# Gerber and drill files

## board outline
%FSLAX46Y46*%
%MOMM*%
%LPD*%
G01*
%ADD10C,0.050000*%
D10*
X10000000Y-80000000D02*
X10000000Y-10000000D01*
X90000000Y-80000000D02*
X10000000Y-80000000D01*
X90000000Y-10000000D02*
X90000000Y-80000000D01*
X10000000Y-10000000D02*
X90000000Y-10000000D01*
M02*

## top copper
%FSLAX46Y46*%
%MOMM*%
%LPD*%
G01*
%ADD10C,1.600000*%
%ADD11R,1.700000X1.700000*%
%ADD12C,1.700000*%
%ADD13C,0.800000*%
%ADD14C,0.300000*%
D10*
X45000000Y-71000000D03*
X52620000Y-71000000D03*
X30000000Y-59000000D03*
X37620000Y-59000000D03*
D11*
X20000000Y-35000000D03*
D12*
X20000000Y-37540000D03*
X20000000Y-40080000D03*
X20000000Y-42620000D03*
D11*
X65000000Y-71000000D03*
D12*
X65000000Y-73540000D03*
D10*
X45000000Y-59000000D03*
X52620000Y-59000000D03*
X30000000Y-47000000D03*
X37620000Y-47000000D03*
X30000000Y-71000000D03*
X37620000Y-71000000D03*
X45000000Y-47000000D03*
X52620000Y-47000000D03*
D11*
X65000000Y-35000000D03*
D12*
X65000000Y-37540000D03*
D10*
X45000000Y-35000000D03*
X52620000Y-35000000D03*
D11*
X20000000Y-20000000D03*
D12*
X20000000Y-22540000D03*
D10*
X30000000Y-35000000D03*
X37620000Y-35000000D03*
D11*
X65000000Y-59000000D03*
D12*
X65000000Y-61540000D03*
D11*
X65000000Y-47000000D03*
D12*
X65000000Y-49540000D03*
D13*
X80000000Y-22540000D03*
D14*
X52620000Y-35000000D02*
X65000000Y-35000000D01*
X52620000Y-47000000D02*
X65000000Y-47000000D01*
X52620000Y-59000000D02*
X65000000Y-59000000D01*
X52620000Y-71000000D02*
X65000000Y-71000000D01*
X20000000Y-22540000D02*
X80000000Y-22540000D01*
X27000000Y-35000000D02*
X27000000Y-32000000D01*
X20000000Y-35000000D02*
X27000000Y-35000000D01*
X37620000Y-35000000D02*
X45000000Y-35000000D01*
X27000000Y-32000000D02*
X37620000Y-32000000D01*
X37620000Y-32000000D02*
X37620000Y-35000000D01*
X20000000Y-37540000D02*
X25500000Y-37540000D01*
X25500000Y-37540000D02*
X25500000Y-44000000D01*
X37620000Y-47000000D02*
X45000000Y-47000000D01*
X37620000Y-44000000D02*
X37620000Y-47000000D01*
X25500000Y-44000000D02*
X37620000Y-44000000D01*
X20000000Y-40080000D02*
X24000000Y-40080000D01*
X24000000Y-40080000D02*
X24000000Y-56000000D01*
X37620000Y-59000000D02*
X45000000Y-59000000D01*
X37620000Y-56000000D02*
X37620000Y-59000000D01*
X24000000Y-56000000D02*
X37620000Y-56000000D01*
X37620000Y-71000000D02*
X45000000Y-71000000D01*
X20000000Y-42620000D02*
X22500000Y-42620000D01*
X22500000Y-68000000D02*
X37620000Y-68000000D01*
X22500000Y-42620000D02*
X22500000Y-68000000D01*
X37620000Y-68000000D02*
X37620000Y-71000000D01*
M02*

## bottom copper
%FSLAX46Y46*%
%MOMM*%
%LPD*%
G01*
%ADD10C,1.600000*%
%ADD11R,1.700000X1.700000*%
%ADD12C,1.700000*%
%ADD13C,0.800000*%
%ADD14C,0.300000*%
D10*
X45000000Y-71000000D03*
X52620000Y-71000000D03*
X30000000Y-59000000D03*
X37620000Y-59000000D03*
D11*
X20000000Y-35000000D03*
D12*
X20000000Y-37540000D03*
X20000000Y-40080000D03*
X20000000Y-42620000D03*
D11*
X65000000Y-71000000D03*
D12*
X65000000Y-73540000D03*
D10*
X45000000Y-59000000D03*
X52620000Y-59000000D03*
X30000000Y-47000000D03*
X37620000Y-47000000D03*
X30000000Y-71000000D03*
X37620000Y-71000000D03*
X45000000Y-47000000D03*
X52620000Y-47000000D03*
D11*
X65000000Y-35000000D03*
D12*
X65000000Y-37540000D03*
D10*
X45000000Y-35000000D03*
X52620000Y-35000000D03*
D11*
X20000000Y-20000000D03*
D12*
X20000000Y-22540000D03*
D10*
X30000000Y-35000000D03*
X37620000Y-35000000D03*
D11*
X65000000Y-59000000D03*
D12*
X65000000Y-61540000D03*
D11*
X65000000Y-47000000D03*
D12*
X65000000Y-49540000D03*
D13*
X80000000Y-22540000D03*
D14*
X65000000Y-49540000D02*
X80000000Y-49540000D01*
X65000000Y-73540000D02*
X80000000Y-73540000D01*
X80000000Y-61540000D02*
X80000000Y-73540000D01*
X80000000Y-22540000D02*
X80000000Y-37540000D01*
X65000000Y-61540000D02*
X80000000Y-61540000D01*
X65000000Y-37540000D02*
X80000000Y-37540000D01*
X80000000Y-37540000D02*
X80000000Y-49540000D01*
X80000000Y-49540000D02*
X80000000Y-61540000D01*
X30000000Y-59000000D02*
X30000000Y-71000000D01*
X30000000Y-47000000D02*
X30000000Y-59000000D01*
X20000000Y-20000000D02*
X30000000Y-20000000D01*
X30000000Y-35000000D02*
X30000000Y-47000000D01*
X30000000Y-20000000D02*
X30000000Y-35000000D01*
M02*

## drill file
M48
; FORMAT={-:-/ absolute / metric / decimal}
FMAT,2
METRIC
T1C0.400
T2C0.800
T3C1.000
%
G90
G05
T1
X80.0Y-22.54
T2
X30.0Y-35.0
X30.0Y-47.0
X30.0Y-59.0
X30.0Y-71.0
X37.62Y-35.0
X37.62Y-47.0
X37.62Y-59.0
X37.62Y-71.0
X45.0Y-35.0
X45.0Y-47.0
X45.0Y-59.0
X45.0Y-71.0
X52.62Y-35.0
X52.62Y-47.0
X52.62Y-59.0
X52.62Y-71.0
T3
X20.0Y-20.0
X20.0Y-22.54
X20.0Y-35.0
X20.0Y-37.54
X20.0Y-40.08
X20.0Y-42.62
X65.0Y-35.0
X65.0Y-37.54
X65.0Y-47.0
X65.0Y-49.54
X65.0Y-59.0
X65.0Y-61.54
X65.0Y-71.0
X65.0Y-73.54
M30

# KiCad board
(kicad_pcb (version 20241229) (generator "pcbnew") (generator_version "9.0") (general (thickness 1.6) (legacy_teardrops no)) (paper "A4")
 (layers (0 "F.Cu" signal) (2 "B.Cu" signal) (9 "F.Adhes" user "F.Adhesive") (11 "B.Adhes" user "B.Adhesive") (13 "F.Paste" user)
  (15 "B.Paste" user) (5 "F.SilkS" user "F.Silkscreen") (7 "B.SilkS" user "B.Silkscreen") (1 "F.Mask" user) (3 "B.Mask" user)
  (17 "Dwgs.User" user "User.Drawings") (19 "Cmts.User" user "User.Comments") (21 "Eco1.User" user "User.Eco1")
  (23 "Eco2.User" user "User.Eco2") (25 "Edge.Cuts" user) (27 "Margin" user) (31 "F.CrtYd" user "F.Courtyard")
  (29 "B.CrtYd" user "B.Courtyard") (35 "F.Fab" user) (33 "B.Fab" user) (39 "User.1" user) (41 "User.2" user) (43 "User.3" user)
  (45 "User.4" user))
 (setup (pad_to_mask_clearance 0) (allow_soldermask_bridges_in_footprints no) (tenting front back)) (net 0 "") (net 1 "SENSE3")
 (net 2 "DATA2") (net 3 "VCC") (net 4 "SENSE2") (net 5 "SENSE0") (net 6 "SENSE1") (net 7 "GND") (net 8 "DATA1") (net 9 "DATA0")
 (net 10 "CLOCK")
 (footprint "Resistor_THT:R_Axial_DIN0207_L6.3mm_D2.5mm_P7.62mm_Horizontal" (layer "F.Cu") (at 45 71)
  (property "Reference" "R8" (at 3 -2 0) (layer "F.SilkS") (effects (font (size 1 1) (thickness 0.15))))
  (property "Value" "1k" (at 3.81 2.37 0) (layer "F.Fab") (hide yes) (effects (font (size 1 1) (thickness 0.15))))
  (pad "1" thru_hole circle (at 0 0) (size 1.6 1.6) (drill 0.8) (layers "*.Cu" "*.Mask") (remove_unused_layers no) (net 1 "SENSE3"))
  (pad "2" thru_hole circle (at 7.62 0) (size 1.6 1.6) (drill 0.8) (layers "*.Cu" "*.Mask") (remove_unused_layers no) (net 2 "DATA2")))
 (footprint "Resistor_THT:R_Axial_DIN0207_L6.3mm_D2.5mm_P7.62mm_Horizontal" (layer "F.Cu") (at 30 59)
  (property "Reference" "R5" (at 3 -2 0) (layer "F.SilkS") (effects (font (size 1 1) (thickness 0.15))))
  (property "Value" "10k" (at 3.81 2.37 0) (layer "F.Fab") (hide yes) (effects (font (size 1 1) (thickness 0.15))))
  (pad "1" thru_hole circle (at 0 0) (size 1.6 1.6) (drill 0.8) (layers "*.Cu" "*.Mask") (remove_unused_layers no) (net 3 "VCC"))
  (pad "2" thru_hole circle (at 7.62 0) (size 1.6 1.6) (drill 0.8) (layers "*.Cu" "*.Mask") (remove_unused_layers no) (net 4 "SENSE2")))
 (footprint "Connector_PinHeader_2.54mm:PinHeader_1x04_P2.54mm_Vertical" (layer "F.Cu") (at 20 35)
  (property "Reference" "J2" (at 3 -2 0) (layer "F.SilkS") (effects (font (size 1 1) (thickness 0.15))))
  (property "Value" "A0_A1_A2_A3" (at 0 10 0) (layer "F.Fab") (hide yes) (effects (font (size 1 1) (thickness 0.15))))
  (pad "1" thru_hole rect (at 0 0) (size 1.7 1.7) (drill 1) (layers "*.Cu" "*.Mask") (remove_unused_layers no) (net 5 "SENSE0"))
  (pad "2" thru_hole circle (at 0 2.54) (size 1.7 1.7) (drill 1) (layers "*.Cu" "*.Mask") (remove_unused_layers no) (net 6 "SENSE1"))
  (pad "3" thru_hole circle (at 0 5.08) (size 1.7 1.7) (drill 1) (layers "*.Cu" "*.Mask") (remove_unused_layers no) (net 4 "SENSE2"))
  (pad "4" thru_hole circle (at 0 7.62) (size 1.7 1.7) (drill 1) (layers "*.Cu" "*.Mask") (remove_unused_layers no) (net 1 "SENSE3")))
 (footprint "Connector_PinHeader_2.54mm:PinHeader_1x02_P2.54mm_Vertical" (layer "F.Cu") (at 65 71)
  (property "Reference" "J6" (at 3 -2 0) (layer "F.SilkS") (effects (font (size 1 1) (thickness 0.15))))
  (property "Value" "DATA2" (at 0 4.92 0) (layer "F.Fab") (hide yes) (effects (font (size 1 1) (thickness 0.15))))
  (pad "1" thru_hole rect (at 0 0) (size 1.7 1.7) (drill 1) (layers "*.Cu" "*.Mask") (remove_unused_layers no) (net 2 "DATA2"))
  (pad "2" thru_hole circle (at 0 2.54) (size 1.7 1.7) (drill 1) (layers "*.Cu" "*.Mask") (remove_unused_layers no) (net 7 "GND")))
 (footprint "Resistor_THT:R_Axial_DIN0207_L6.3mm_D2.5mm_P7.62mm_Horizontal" (layer "F.Cu") (at 45 59)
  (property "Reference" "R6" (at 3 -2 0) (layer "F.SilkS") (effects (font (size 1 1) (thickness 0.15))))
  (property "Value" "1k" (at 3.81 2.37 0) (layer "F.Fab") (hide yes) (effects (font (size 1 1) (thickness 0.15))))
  (pad "1" thru_hole circle (at 0 0) (size 1.6 1.6) (drill 0.8) (layers "*.Cu" "*.Mask") (remove_unused_layers no) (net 4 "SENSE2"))
  (pad "2" thru_hole circle (at 7.62 0) (size 1.6 1.6) (drill 0.8) (layers "*.Cu" "*.Mask") (remove_unused_layers no) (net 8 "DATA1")))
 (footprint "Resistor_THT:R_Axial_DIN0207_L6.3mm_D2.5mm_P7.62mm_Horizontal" (layer "F.Cu") (at 30 47)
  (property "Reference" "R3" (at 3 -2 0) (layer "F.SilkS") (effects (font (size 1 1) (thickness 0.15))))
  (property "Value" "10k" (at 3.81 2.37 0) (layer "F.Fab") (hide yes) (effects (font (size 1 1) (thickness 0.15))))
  (pad "1" thru_hole circle (at 0 0) (size 1.6 1.6) (drill 0.8) (layers "*.Cu" "*.Mask") (remove_unused_layers no) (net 3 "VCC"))
  (pad "2" thru_hole circle (at 7.62 0) (size 1.6 1.6) (drill 0.8) (layers "*.Cu" "*.Mask") (remove_unused_layers no) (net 6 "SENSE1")))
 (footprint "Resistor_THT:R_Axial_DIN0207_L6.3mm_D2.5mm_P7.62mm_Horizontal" (layer "F.Cu") (at 30 71)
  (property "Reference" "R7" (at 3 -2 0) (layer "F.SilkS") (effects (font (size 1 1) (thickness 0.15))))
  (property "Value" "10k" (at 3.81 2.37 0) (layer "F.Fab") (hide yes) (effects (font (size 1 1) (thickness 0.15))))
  (pad "1" thru_hole circle (at 0 0) (size 1.6 1.6) (drill 0.8) (layers "*.Cu" "*.Mask") (remove_unused_layers no) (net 3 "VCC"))
  (pad "2" thru_hole circle (at 7.62 0) (size 1.6 1.6) (drill 0.8) (layers "*.Cu" "*.Mask") (remove_unused_layers no) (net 1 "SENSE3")))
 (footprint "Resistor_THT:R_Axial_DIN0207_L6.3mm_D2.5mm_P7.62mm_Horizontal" (layer "F.Cu") (at 45 47)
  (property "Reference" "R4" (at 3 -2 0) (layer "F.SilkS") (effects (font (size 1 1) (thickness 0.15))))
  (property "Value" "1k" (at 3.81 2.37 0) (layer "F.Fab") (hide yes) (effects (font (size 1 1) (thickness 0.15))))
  (pad "1" thru_hole circle (at 0 0) (size 1.6 1.6) (drill 0.8) (layers "*.Cu" "*.Mask") (remove_unused_layers no) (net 6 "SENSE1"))
  (pad "2" thru_hole circle (at 7.62 0) (size 1.6 1.6) (drill 0.8) (layers "*.Cu" "*.Mask") (remove_unused_layers no) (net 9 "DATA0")))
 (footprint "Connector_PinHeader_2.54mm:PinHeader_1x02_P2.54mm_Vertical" (layer "F.Cu") (at 65 35)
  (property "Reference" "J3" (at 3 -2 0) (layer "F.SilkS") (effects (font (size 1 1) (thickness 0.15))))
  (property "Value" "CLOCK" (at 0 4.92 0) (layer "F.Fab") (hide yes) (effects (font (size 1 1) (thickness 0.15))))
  (pad "1" thru_hole rect (at 0 0) (size 1.7 1.7) (drill 1) (layers "*.Cu" "*.Mask") (remove_unused_layers no) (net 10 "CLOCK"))
  (pad "2" thru_hole circle (at 0 2.54) (size 1.7 1.7) (drill 1) (layers "*.Cu" "*.Mask") (remove_unused_layers no) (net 7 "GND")))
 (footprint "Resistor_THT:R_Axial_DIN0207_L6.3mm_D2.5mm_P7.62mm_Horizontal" (layer "F.Cu") (at 45 35)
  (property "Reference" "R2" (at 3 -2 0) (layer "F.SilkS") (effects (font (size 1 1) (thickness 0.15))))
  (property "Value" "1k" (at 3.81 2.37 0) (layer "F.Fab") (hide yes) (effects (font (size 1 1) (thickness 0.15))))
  (pad "1" thru_hole circle (at 0 0) (size 1.6 1.6) (drill 0.8) (layers "*.Cu" "*.Mask") (remove_unused_layers no) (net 5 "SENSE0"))
  (pad "2" thru_hole circle (at 7.62 0) (size 1.6 1.6) (drill 0.8) (layers "*.Cu" "*.Mask") (remove_unused_layers no) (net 10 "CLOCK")))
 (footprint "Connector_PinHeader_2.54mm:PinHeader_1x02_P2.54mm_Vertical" (layer "F.Cu") (at 20 20)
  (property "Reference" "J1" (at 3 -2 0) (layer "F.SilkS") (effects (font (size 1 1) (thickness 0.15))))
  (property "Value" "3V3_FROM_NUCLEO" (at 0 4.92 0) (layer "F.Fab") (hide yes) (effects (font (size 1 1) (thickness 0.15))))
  (pad "1" thru_hole rect (at 0 0) (size 1.7 1.7) (drill 1) (layers "*.Cu" "*.Mask") (remove_unused_layers no) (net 3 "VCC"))
  (pad "2" thru_hole circle (at 0 2.54) (size 1.7 1.7) (drill 1) (layers "*.Cu" "*.Mask") (remove_unused_layers no) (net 7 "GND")))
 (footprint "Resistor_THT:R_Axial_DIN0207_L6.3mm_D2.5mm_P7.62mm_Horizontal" (layer "F.Cu") (at 30 35)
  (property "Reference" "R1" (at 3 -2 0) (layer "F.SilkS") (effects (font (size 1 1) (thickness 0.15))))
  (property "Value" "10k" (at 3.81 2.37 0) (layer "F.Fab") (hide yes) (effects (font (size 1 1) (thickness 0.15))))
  (pad "1" thru_hole circle (at 0 0) (size 1.6 1.6) (drill 0.8) (layers "*.Cu" "*.Mask") (remove_unused_layers no) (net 3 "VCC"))
  (pad "2" thru_hole circle (at 7.62 0) (size 1.6 1.6) (drill 0.8) (layers "*.Cu" "*.Mask") (remove_unused_layers no) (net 5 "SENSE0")))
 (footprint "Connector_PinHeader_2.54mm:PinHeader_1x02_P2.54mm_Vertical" (layer "F.Cu") (at 65 59)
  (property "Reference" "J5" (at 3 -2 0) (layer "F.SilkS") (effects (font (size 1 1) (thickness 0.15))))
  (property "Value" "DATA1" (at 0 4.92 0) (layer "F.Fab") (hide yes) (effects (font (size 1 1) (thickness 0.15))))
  (pad "1" thru_hole rect (at 0 0) (size 1.7 1.7) (drill 1) (layers "*.Cu" "*.Mask") (remove_unused_layers no) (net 8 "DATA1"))
  (pad "2" thru_hole circle (at 0 2.54) (size 1.7 1.7) (drill 1) (layers "*.Cu" "*.Mask") (remove_unused_layers no) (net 7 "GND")))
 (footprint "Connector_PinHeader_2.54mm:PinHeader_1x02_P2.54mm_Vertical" (layer "F.Cu") (at 65 47)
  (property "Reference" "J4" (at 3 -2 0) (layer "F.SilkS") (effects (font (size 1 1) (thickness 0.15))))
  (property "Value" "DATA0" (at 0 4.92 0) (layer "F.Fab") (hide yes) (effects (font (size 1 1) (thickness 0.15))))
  (pad "1" thru_hole rect (at 0 0) (size 1.7 1.7) (drill 1) (layers "*.Cu" "*.Mask") (remove_unused_layers no) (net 9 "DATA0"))
  (pad "2" thru_hole circle (at 0 2.54) (size 1.7 1.7) (drill 1) (layers "*.Cu" "*.Mask") (remove_unused_layers no) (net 7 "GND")))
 (gr_line (start 10 80) (end 10 10) (stroke (width 0.05) (type default)) (layer "Edge.Cuts"))
 (gr_line (start 90 80) (end 10 80) (stroke (width 0.05) (type default)) (layer "Edge.Cuts"))
 (gr_line (start 90 10) (end 90 80) (stroke (width 0.05) (type default)) (layer "Edge.Cuts"))
 (gr_line (start 10 10) (end 90 10) (stroke (width 0.05) (type default)) (layer "Edge.Cuts"))
 (segment (start 52.62 35) (end 65 35) (width 0.3) (layer "F.Cu") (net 10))
 (segment (start 52.62 47) (end 65 47) (width 0.3) (layer "F.Cu") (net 9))
 (segment (start 52.62 59) (end 65 59) (width 0.3) (layer "F.Cu") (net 8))
 (segment (start 52.62 71) (end 65 71) (width 0.3) (layer "F.Cu") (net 2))
 (segment (start 20 22.54) (end 80 22.54) (width 0.3) (layer "F.Cu") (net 7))
 (via (at 80 22.54) (size 0.8) (drill 0.4) (layers "F.Cu" "B.Cu") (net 7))
 (segment (start 65 49.54) (end 80 49.54) (width 0.3) (layer "B.Cu") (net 7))
 (segment (start 65 73.54) (end 80 73.54) (width 0.3) (layer "B.Cu") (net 7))
 (segment (start 80 61.54) (end 80 73.54) (width 0.3) (layer "B.Cu") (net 7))
 (segment (start 80 22.54) (end 80 37.54) (width 0.3) (layer "B.Cu") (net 7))
 (segment (start 65 61.54) (end 80 61.54) (width 0.3) (layer "B.Cu") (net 7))
 (segment (start 65 37.54) (end 80 37.54) (width 0.3) (layer "B.Cu") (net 7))
 (segment (start 80 37.54) (end 80 49.54) (width 0.3) (layer "B.Cu") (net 7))
 (segment (start 80 49.54) (end 80 61.54) (width 0.3) (layer "B.Cu") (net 7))
 (segment (start 27 35) (end 27 32) (width 0.3) (layer "F.Cu") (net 5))
 (segment (start 20 35) (end 27 35) (width 0.3) (layer "F.Cu") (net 5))
 (segment (start 37.62 35) (end 45 35) (width 0.3) (layer "F.Cu") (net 5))
 (segment (start 27 32) (end 37.62 32) (width 0.3) (layer "F.Cu") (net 5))
 (segment (start 37.62 32) (end 37.62 35) (width 0.3) (layer "F.Cu") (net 5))
 (segment (start 20 37.54) (end 25.5 37.54) (width 0.3) (layer "F.Cu") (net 6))
 (segment (start 25.5 37.54) (end 25.5 44) (width 0.3) (layer "F.Cu") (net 6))
 (segment (start 37.62 47) (end 45 47) (width 0.3) (layer "F.Cu") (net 6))
 (segment (start 37.62 44) (end 37.62 47) (width 0.3) (layer "F.Cu") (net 6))
 (segment (start 25.5 44) (end 37.62 44) (width 0.3) (layer "F.Cu") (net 6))
 (segment (start 20 40.08) (end 24 40.08) (width 0.3) (layer "F.Cu") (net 4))
 (segment (start 24 40.08) (end 24 56) (width 0.3) (layer "F.Cu") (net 4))
 (segment (start 37.62 59) (end 45 59) (width 0.3) (layer "F.Cu") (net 4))
 (segment (start 37.62 56) (end 37.62 59) (width 0.3) (layer "F.Cu") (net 4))
 (segment (start 24 56) (end 37.62 56) (width 0.3) (layer "F.Cu") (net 4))
 (segment (start 37.62 71) (end 45 71) (width 0.3) (layer "F.Cu") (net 1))
 (segment (start 20 42.62) (end 22.5 42.62) (width 0.3) (layer "F.Cu") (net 1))
 (segment (start 22.5 68) (end 37.62 68) (width 0.3) (layer "F.Cu") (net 1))
 (segment (start 22.5 42.62) (end 22.5 68) (width 0.3) (layer "F.Cu") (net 1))
 (segment (start 37.62 68) (end 37.62 71) (width 0.3) (layer "F.Cu") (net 1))
 (segment (start 30 59) (end 30 71) (width 0.3) (layer "B.Cu") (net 3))
 (segment (start 30 47) (end 30 59) (width 0.3) (layer "B.Cu") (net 3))
 (segment (start 20 20) (end 30 20) (width 0.3) (layer "B.Cu") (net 3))
 (segment (start 30 35) (end 30 47) (width 0.3) (layer "B.Cu") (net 3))
 (segment (start 30 20) (end 30 35) (width 0.3) (layer "B.Cu") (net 3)))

